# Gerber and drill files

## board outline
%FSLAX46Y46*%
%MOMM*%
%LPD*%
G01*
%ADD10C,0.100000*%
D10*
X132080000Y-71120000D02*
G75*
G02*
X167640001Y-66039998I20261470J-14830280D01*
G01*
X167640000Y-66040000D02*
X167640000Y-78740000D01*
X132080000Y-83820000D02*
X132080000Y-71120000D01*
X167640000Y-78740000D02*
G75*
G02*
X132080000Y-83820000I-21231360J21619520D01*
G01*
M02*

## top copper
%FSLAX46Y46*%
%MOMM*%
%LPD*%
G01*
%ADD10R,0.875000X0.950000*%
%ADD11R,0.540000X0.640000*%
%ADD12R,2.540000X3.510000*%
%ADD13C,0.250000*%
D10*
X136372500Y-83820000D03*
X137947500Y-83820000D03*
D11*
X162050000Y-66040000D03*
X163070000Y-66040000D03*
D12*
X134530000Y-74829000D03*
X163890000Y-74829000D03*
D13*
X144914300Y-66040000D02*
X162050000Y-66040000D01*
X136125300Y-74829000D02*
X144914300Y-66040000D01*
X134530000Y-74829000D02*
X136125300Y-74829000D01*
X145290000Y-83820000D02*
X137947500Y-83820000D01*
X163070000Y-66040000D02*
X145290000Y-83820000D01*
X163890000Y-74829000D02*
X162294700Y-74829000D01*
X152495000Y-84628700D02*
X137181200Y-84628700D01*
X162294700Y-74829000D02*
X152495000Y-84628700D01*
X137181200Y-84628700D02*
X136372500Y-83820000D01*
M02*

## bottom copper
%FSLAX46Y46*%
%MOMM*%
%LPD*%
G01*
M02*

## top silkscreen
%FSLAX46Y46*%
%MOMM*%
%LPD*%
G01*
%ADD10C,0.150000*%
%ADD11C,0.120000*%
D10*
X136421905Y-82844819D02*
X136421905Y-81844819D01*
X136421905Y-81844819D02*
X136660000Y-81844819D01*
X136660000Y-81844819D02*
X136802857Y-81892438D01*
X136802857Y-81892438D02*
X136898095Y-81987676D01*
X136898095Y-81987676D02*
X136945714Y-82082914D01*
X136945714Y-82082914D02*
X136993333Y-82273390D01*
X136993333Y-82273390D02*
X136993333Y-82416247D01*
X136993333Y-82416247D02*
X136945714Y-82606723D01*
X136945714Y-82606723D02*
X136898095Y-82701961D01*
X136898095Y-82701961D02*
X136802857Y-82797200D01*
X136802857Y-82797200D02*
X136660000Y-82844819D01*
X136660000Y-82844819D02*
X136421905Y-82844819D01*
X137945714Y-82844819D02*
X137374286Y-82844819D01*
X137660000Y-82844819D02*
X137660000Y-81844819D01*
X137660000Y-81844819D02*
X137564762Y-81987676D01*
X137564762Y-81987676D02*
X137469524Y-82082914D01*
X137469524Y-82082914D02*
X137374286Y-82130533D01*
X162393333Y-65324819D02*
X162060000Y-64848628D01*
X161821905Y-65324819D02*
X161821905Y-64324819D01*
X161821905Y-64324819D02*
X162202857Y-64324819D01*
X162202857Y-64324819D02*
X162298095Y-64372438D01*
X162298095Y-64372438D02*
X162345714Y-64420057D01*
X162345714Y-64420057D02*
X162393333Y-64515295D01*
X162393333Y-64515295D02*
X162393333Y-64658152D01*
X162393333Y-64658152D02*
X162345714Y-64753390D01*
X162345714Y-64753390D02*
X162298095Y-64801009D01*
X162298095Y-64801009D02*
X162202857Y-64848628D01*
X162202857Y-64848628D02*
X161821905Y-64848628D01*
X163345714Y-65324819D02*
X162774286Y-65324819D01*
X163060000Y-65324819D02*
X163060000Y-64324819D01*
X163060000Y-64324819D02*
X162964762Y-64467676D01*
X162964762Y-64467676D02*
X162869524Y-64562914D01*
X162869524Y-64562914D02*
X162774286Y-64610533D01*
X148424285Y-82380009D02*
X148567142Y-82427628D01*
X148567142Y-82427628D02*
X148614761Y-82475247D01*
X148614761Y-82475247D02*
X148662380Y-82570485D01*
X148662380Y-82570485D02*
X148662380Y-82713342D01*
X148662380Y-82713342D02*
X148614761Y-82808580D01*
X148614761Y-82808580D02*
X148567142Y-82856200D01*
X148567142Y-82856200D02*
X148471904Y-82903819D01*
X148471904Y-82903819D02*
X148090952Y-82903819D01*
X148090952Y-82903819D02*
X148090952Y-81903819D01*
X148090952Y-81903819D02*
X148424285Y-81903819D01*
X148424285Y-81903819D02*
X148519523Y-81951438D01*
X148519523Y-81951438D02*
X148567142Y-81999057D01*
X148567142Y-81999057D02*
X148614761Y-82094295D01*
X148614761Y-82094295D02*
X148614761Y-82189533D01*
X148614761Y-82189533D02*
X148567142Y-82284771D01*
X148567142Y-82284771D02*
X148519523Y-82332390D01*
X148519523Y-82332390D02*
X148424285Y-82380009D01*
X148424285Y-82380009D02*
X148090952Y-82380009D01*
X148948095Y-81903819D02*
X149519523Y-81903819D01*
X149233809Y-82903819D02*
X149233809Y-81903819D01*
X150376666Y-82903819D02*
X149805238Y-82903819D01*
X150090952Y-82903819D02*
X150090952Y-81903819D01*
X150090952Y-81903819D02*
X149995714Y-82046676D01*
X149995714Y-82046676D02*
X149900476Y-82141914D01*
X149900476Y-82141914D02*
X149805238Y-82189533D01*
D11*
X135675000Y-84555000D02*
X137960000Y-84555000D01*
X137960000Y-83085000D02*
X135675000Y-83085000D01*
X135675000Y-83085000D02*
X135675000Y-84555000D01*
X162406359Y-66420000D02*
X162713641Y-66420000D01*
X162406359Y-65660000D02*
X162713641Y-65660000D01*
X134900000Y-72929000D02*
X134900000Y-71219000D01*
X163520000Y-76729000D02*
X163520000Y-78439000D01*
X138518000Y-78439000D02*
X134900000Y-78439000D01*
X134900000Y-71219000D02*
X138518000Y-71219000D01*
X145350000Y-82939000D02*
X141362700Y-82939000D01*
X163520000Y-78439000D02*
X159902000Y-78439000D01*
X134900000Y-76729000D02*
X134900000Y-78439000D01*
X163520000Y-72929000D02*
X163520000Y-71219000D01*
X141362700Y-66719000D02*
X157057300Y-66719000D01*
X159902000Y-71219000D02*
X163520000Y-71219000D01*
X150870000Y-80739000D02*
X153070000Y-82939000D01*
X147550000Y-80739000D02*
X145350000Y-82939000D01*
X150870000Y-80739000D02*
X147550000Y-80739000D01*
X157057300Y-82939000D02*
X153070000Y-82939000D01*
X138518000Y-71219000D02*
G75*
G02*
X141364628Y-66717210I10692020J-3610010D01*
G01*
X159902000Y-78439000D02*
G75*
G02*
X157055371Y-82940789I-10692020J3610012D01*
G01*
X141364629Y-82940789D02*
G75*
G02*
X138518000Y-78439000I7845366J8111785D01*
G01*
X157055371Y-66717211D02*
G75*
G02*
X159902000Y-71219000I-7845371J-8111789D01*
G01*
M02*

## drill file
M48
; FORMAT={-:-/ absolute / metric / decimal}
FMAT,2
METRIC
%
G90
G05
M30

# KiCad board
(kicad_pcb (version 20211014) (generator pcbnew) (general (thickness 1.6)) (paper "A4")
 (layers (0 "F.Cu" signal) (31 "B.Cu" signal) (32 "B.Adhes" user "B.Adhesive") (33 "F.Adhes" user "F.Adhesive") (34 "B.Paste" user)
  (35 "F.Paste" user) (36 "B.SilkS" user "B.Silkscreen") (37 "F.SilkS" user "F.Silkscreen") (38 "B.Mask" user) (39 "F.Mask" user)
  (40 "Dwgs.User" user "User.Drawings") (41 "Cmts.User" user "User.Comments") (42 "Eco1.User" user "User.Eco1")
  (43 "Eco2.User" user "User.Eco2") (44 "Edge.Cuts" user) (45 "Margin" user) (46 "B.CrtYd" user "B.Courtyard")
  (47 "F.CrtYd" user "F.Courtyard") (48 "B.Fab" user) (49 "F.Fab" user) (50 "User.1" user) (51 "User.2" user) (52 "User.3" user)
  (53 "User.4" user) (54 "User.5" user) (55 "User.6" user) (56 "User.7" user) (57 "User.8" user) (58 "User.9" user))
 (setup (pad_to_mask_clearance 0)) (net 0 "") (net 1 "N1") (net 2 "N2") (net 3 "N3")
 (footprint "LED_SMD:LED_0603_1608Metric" (layer "F.Cu") (at 137.16 83.82)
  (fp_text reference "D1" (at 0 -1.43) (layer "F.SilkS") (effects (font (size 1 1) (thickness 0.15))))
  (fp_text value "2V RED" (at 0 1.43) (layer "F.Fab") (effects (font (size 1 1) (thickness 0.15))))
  (fp_line (start -1.485 0.735) (end 0.8 0.735) (layer "F.SilkS") (width 0.12))
  (fp_line (start 0.8 -0.735) (end -1.485 -0.735) (layer "F.SilkS") (width 0.12))
  (fp_line (start -1.485 -0.735) (end -1.485 0.735) (layer "F.SilkS") (width 0.12))
  (pad "1" smd rect (at -0.7875 0) (size 0.875 0.95) (layers "F.Cu" "F.Paste" "F.Mask") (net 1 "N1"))
  (pad "2" smd rect (at 0.7875 0) (size 0.875 0.95) (layers "F.Cu" "F.Paste" "F.Mask") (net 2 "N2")))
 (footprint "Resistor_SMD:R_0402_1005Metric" (layer "F.Cu") (at 162.56 66.04)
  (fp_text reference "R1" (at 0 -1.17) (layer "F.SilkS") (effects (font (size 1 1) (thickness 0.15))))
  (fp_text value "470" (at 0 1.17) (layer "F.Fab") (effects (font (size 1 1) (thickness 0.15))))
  (fp_line (start -0.153641 0.38) (end 0.153641 0.38) (layer "F.SilkS") (width 0.12))
  (fp_line (start -0.153641 -0.38) (end 0.153641 -0.38) (layer "F.SilkS") (width 0.12))
  (pad "1" smd rect (at -0.51 0) (size 0.54 0.64) (layers "F.Cu" "F.Paste" "F.Mask") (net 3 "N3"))
  (pad "2" smd rect (at 0.51 0) (size 0.54 0.64) (layers "F.Cu" "F.Paste" "F.Mask") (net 2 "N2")))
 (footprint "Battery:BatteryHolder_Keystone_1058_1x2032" (layer "F.Cu") (at 149.21 74.829)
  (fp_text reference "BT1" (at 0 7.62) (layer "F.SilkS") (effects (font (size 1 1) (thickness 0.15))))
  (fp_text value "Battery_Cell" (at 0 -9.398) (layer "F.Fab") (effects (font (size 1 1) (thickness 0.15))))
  (fp_line (start -14.31 -1.9) (end -14.31 -3.61) (layer "F.SilkS") (width 0.12))
  (fp_line (start 14.31 1.9) (end 14.31 3.61) (layer "F.SilkS") (width 0.12))
  (fp_line (start -10.692 3.61) (end -14.31 3.61) (layer "F.SilkS") (width 0.12))
  (fp_line (start -14.31 -3.61) (end -10.692 -3.61) (layer "F.SilkS") (width 0.12))
  (fp_line (start -3.86 8.11) (end -7.8473 8.11) (layer "F.SilkS") (width 0.12))
  (fp_line (start 14.31 3.61) (end 10.692 3.61) (layer "F.SilkS") (width 0.12))
  (fp_line (start -14.31 1.9) (end -14.31 3.61) (layer "F.SilkS") (width 0.12))
  (fp_line (start 14.31 -1.9) (end 14.31 -3.61) (layer "F.SilkS") (width 0.12))
  (fp_line (start -7.8473 -8.11) (end 7.8473 -8.11) (layer "F.SilkS") (width 0.12))
  (fp_line (start 10.692 -3.61) (end 14.31 -3.61) (layer "F.SilkS") (width 0.12))
  (fp_line (start 1.66 5.91) (end 3.86 8.11) (layer "F.SilkS") (width 0.12))
  (fp_line (start -1.66 5.91) (end -3.86 8.11) (layer "F.SilkS") (width 0.12))
  (fp_line (start 1.66 5.91) (end -1.66 5.91) (layer "F.SilkS") (width 0.12))
  (fp_line (start 7.8473 8.11) (end 3.86 8.11) (layer "F.SilkS") (width 0.12))
  (fp_arc (start -10.692 -3.61) (mid -9.538084 -6.031244) (end -7.845371 -8.111789) (layer "F.SilkS") (width 0.12))
  (fp_arc (start 10.692 3.61) (mid 9.538084 6.031244) (end 7.845371 8.111789) (layer "F.SilkS") (width 0.12))
  (fp_arc (start -7.845371 8.111789) (mid -9.538085 6.031244) (end -10.692 3.61) (layer "F.SilkS") (width 0.12))
  (fp_arc (start 7.845371 -8.111789) (mid 9.538085 -6.031244) (end 10.692 -3.61) (layer "F.SilkS") (width 0.12))
  (pad "1" smd rect (at -14.68 0) (size 2.54 3.51) (layers "F.Cu" "F.Paste" "F.Mask") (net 3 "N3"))
  (pad "2" smd rect (at 14.68 0) (size 2.54 3.51) (layers "F.Cu" "F.Paste" "F.Mask") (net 1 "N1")))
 (gr_arc (start 132.08 71.12) (mid 148.790513 61.093589) (end 167.64 66.04) (layer "Edge.Cuts") (width 0.1))
 (gr_line (start 167.64 66.04) (end 167.64 78.74) (layer "Edge.Cuts") (width 0.1))
 (gr_line (start 132.08 83.82) (end 132.08 71.12) (layer "Edge.Cuts") (width 0.1))
 (gr_arc (start 167.64 78.74) (mid 150.693904 87.117326) (end 132.08 83.82) (layer "Edge.Cuts") (width 0.1))
 (segment (start 144.9143 66.04) (end 162.05 66.04) (width 0.25) (layer "F.Cu") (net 3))
 (segment (start 136.1253 74.829) (end 144.9143 66.04) (width 0.25) (layer "F.Cu") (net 3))
 (segment (start 134.53 74.829) (end 136.1253 74.829) (width 0.25) (layer "F.Cu") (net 3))
 (segment (start 145.29 83.82) (end 137.9475 83.82) (width 0.25) (layer "F.Cu") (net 2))
 (segment (start 163.07 66.04) (end 145.29 83.82) (width 0.25) (layer "F.Cu") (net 2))
 (segment (start 163.89 74.829) (end 162.2947 74.829) (width 0.25) (layer "F.Cu") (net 1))
 (segment (start 152.495 84.6287) (end 137.1812 84.6287) (width 0.25) (layer "F.Cu") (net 1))
 (segment (start 162.2947 74.829) (end 152.495 84.6287) (width 0.25) (layer "F.Cu") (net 1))
 (segment (start 137.1812 84.6287) (end 136.3725 83.82) (width 0.25) (layer "F.Cu") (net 1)))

